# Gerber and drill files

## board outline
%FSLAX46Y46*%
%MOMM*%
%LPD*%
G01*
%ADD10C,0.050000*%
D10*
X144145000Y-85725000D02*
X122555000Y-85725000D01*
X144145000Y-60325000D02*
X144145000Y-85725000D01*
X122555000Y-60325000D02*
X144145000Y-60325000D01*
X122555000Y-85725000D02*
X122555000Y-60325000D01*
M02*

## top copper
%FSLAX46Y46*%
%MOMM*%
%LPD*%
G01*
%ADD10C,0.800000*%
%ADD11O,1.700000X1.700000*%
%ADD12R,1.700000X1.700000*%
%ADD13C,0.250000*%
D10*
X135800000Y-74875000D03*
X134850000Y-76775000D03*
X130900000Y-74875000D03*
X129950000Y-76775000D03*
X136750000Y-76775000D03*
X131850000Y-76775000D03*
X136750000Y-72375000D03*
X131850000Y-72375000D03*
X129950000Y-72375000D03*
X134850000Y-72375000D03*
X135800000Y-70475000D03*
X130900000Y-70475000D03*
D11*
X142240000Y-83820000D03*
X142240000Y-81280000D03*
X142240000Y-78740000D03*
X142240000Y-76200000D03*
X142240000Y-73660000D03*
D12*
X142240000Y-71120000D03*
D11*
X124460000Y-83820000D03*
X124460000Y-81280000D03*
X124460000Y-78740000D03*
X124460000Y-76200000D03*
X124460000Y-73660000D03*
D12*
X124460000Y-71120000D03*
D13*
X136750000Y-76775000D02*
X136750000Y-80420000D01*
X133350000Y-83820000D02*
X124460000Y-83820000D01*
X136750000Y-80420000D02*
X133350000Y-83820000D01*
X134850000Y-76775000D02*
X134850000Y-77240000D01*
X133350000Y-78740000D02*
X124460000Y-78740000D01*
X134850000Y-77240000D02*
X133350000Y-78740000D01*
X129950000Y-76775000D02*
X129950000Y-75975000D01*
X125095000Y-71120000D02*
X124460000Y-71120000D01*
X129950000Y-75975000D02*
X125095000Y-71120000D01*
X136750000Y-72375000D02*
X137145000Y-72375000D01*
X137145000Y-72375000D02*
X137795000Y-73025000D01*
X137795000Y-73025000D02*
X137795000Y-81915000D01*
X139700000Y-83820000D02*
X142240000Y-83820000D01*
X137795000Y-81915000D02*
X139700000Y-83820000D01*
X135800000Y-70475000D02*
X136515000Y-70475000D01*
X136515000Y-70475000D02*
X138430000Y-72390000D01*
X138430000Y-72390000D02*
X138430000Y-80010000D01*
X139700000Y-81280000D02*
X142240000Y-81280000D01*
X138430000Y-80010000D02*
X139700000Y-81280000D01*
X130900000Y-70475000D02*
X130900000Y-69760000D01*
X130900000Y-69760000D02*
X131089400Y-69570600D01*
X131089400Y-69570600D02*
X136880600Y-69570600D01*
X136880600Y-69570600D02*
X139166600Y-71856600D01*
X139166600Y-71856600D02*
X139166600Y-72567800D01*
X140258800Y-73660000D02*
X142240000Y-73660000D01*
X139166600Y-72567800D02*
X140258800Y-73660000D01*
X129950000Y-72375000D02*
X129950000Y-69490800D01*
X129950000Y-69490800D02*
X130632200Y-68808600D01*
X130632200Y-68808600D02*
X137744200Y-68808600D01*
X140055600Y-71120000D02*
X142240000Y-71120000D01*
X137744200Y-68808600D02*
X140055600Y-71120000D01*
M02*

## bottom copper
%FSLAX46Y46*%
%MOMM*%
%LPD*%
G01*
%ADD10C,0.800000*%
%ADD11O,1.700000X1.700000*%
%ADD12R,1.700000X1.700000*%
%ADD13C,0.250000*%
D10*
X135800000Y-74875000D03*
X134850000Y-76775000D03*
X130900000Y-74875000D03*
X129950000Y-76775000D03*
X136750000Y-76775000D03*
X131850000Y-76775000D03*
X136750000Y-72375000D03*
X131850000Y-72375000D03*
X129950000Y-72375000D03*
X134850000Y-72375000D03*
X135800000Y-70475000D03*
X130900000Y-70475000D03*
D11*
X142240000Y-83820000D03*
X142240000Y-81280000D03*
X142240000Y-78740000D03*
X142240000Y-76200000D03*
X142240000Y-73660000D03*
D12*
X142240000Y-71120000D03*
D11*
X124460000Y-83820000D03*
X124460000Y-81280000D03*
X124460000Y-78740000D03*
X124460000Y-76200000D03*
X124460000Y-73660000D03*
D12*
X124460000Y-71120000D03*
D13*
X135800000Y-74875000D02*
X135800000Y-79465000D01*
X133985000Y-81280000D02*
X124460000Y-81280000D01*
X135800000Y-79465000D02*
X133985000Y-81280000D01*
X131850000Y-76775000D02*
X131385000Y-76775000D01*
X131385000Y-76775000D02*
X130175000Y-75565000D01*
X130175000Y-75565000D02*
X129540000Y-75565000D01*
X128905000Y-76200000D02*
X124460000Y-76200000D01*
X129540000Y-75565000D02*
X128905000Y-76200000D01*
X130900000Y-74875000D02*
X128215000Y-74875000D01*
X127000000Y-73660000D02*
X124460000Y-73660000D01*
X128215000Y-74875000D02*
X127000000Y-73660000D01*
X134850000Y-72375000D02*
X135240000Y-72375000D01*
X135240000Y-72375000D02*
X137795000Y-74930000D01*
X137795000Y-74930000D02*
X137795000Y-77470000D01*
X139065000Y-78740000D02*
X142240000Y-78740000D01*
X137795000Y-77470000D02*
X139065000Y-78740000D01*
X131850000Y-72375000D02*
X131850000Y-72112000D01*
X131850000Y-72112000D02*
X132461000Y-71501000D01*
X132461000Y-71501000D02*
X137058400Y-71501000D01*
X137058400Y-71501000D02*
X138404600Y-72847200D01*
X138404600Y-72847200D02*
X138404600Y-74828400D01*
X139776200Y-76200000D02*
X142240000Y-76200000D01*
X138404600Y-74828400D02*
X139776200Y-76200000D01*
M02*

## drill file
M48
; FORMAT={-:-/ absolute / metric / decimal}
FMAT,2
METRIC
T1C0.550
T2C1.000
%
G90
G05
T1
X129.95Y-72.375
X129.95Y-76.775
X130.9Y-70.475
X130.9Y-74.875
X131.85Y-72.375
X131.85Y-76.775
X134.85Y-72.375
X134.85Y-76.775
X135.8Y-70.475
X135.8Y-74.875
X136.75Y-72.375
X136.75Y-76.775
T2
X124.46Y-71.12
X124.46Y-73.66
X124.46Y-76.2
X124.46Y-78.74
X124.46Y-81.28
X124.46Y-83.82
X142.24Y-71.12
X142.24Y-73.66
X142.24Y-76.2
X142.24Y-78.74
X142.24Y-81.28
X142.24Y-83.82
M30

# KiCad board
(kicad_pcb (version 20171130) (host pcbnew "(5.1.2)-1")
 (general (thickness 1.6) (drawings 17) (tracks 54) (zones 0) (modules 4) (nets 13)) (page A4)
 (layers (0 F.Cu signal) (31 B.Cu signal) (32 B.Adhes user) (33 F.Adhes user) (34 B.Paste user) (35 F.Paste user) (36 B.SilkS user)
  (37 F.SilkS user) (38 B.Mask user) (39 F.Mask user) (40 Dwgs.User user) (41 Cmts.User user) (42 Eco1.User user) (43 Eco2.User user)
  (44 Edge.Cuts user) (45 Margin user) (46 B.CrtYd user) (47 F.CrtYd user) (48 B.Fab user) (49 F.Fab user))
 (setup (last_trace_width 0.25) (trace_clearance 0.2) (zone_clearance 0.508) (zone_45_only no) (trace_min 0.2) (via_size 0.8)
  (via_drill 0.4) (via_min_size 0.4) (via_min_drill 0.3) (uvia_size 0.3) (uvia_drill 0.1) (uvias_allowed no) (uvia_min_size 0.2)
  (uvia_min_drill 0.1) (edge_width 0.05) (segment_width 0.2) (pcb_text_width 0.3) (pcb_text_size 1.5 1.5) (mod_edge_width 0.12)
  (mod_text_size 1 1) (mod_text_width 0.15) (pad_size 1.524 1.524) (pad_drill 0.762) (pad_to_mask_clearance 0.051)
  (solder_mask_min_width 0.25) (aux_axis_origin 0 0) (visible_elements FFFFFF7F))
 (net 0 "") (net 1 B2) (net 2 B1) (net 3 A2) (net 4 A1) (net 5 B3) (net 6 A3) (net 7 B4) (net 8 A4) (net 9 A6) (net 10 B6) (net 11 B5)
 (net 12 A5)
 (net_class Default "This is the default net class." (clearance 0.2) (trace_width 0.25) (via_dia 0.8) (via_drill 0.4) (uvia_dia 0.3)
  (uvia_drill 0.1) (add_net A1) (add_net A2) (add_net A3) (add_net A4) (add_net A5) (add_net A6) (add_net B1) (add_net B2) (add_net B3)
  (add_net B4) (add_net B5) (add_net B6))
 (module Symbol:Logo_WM (layer F.Cu) (at 125.095 64.77 270)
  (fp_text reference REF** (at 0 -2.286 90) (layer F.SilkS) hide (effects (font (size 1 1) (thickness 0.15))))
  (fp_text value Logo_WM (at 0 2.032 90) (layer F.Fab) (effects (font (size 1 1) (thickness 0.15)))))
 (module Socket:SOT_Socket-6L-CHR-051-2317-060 (layer F.Cu) (at 133.35 73.025)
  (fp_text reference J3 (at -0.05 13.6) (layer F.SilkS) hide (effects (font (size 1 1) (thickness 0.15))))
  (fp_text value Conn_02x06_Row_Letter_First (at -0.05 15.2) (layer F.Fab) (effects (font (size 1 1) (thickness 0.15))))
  (pad b2 thru_hole circle (at 2.45 1.85) (size 0.8 0.8) (drill 0.55) (layers *.Cu *.Mask) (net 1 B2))
  (pad b1 thru_hole circle (at 1.5 3.75) (size 0.8 0.8) (drill 0.55) (layers *.Cu *.Mask) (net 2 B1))
  (pad a2 thru_hole circle (at -2.45 1.85) (size 0.8 0.8) (drill 0.55) (layers *.Cu *.Mask) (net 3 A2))
  (pad a1 thru_hole circle (at -3.4 3.75) (size 0.8 0.8) (drill 0.55) (layers *.Cu *.Mask) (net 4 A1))
  (pad b3 thru_hole circle (at 3.4 3.75) (size 0.8 0.8) (drill 0.55) (layers *.Cu *.Mask) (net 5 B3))
  (pad a3 thru_hole circle (at -1.5 3.75) (size 0.8 0.8) (drill 0.55) (layers *.Cu *.Mask) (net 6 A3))
  (pad b4 thru_hole circle (at 3.4 -0.65) (size 0.8 0.8) (drill 0.55) (layers *.Cu *.Mask) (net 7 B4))
  (pad a4 thru_hole circle (at -1.5 -0.65) (size 0.8 0.8) (drill 0.55) (layers *.Cu *.Mask) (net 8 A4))
  (pad a6 thru_hole circle (at -3.4 -0.65) (size 0.8 0.8) (drill 0.55) (layers *.Cu *.Mask) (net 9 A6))
  (pad b6 thru_hole circle (at 1.5 -0.65) (size 0.8 0.8) (drill 0.55) (layers *.Cu *.Mask) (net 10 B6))
  (pad b5 thru_hole circle (at 2.45 -2.55) (size 0.8 0.8) (drill 0.55) (layers *.Cu *.Mask) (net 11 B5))
  (pad a5 thru_hole circle (at -2.45 -2.55) (size 0.8 0.8) (drill 0.55) (layers *.Cu *.Mask) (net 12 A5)))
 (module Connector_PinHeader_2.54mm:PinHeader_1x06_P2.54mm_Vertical (layer B.Cu) (at 142.24 71.12 180)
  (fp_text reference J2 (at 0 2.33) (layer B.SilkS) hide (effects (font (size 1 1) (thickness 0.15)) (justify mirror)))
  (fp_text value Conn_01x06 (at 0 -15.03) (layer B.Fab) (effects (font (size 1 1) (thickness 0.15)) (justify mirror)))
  (pad 6 thru_hole oval (at 0 -12.7 180) (size 1.7 1.7) (drill 1) (layers *.Cu *.Mask) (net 7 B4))
  (pad 5 thru_hole oval (at 0 -10.16 180) (size 1.7 1.7) (drill 1) (layers *.Cu *.Mask) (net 11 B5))
  (pad 4 thru_hole oval (at 0 -7.62 180) (size 1.7 1.7) (drill 1) (layers *.Cu *.Mask) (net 10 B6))
  (pad 3 thru_hole oval (at 0 -5.08 180) (size 1.7 1.7) (drill 1) (layers *.Cu *.Mask) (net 8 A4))
  (pad 2 thru_hole oval (at 0 -2.54 180) (size 1.7 1.7) (drill 1) (layers *.Cu *.Mask) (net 12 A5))
  (pad 1 thru_hole rect (at 0 0 180) (size 1.7 1.7) (drill 1) (layers *.Cu *.Mask) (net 9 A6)))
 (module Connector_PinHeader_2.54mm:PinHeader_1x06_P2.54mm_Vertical (layer B.Cu) (at 124.46 71.12 180)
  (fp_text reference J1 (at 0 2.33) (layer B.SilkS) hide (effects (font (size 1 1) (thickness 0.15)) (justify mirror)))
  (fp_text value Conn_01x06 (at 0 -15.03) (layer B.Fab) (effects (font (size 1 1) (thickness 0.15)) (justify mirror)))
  (pad 6 thru_hole oval (at 0 -12.7 180) (size 1.7 1.7) (drill 1) (layers *.Cu *.Mask) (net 5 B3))
  (pad 5 thru_hole oval (at 0 -10.16 180) (size 1.7 1.7) (drill 1) (layers *.Cu *.Mask) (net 1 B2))
  (pad 4 thru_hole oval (at 0 -7.62 180) (size 1.7 1.7) (drill 1) (layers *.Cu *.Mask) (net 2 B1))
  (pad 3 thru_hole oval (at 0 -5.08 180) (size 1.7 1.7) (drill 1) (layers *.Cu *.Mask) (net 6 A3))
  (pad 2 thru_hole oval (at 0 -2.54 180) (size 1.7 1.7) (drill 1) (layers *.Cu *.Mask) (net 3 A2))
  (pad 1 thru_hole rect (at 0 0 180) (size 1.7 1.7) (drill 1) (layers *.Cu *.Mask) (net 4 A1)))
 (gr_line (start 144.145 85.725) (end 122.555 85.725) (layer Edge.Cuts) (width 0.05))
 (gr_line (start 144.145 60.325) (end 144.145 85.725) (layer Edge.Cuts) (width 0.05))
 (gr_line (start 122.555 60.325) (end 144.145 60.325) (layer Edge.Cuts) (width 0.05))
 (gr_line (start 122.555 85.725) (end 122.555 60.325) (layer Edge.Cuts) (width 0.05))
 (segment (start 136.75 76.775) (end 136.75 80.42) (width 0.25) (layer F.Cu) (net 5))
 (segment (start 133.35 83.82) (end 124.46 83.82) (width 0.25) (layer F.Cu) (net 5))
 (segment (start 136.75 80.42) (end 133.35 83.82) (width 0.25) (layer F.Cu) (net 5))
 (segment (start 135.8 74.875) (end 135.8 79.465) (width 0.25) (layer B.Cu) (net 1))
 (segment (start 133.985 81.28) (end 124.46 81.28) (width 0.25) (layer B.Cu) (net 1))
 (segment (start 135.8 79.465) (end 133.985 81.28) (width 0.25) (layer B.Cu) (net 1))
 (segment (start 134.85 76.775) (end 134.85 77.24) (width 0.25) (layer F.Cu) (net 2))
 (segment (start 133.35 78.74) (end 124.46 78.74) (width 0.25) (layer F.Cu) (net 2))
 (segment (start 134.85 77.24) (end 133.35 78.74) (width 0.25) (layer F.Cu) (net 2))
 (segment (start 131.85 76.775) (end 131.385 76.775) (width 0.25) (layer B.Cu) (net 6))
 (segment (start 131.385 76.775) (end 130.175 75.565) (width 0.25) (layer B.Cu) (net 6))
 (segment (start 130.175 75.565) (end 129.54 75.565) (width 0.25) (layer B.Cu) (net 6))
 (segment (start 128.905 76.2) (end 124.46 76.2) (width 0.25) (layer B.Cu) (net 6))
 (segment (start 129.54 75.565) (end 128.905 76.2) (width 0.25) (layer B.Cu) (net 6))
 (segment (start 130.9 74.875) (end 128.215 74.875) (width 0.25) (layer B.Cu) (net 3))
 (segment (start 127 73.66) (end 124.46 73.66) (width 0.25) (layer B.Cu) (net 3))
 (segment (start 128.215 74.875) (end 127 73.66) (width 0.25) (layer B.Cu) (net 3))
 (segment (start 129.95 76.775) (end 129.95 75.975) (width 0.25) (layer F.Cu) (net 4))
 (segment (start 125.095 71.12) (end 124.46 71.12) (width 0.25) (layer F.Cu) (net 4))
 (segment (start 129.95 75.975) (end 125.095 71.12) (width 0.25) (layer F.Cu) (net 4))
 (segment (start 136.75 72.375) (end 137.145 72.375) (width 0.25) (layer F.Cu) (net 7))
 (segment (start 137.145 72.375) (end 137.795 73.025) (width 0.25) (layer F.Cu) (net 7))
 (segment (start 137.795 73.025) (end 137.795 81.915) (width 0.25) (layer F.Cu) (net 7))
 (segment (start 139.7 83.82) (end 142.24 83.82) (width 0.25) (layer F.Cu) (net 7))
 (segment (start 137.795 81.915) (end 139.7 83.82) (width 0.25) (layer F.Cu) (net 7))
 (segment (start 135.8 70.475) (end 136.515 70.475) (width 0.25) (layer F.Cu) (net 11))
 (segment (start 136.515 70.475) (end 138.43 72.39) (width 0.25) (layer F.Cu) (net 11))
 (segment (start 138.43 72.39) (end 138.43 80.01) (width 0.25) (layer F.Cu) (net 11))
 (segment (start 139.7 81.28) (end 142.24 81.28) (width 0.25) (layer F.Cu) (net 11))
 (segment (start 138.43 80.01) (end 139.7 81.28) (width 0.25) (layer F.Cu) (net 11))
 (segment (start 134.85 72.375) (end 135.24 72.375) (width 0.25) (layer B.Cu) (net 10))
 (segment (start 135.24 72.375) (end 137.795 74.93) (width 0.25) (layer B.Cu) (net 10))
 (segment (start 137.795 74.93) (end 137.795 77.47) (width 0.25) (layer B.Cu) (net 10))
 (segment (start 139.065 78.74) (end 142.24 78.74) (width 0.25) (layer B.Cu) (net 10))
 (segment (start 137.795 77.47) (end 139.065 78.74) (width 0.25) (layer B.Cu) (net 10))
 (segment (start 131.85 72.375) (end 131.85 72.112) (width 0.25) (layer B.Cu) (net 8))
 (segment (start 131.85 72.112) (end 132.461 71.501) (width 0.25) (layer B.Cu) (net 8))
 (segment (start 132.461 71.501) (end 137.0584 71.501) (width 0.25) (layer B.Cu) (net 8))
 (segment (start 137.0584 71.501) (end 138.4046 72.8472) (width 0.25) (layer B.Cu) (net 8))
 (segment (start 138.4046 72.8472) (end 138.4046 74.8284) (width 0.25) (layer B.Cu) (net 8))
 (segment (start 139.7762 76.2) (end 142.24 76.2) (width 0.25) (layer B.Cu) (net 8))
 (segment (start 138.4046 74.8284) (end 139.7762 76.2) (width 0.25) (layer B.Cu) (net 8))
 (segment (start 130.9 70.475) (end 130.9 69.76) (width 0.25) (layer F.Cu) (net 12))
 (segment (start 130.9 69.76) (end 131.0894 69.5706) (width 0.25) (layer F.Cu) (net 12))
 (segment (start 131.0894 69.5706) (end 136.8806 69.5706) (width 0.25) (layer F.Cu) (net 12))
 (segment (start 136.8806 69.5706) (end 139.1666 71.8566) (width 0.25) (layer F.Cu) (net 12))
 (segment (start 139.1666 71.8566) (end 139.1666 72.5678) (width 0.25) (layer F.Cu) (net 12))
 (segment (start 140.2588 73.66) (end 142.24 73.66) (width 0.25) (layer F.Cu) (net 12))
 (segment (start 139.1666 72.5678) (end 140.2588 73.66) (width 0.25) (layer F.Cu) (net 12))
 (segment (start 129.95 72.375) (end 129.95 69.4908) (width 0.25) (layer F.Cu) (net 9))
 (segment (start 129.95 69.4908) (end 130.6322 68.8086) (width 0.25) (layer F.Cu) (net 9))
 (segment (start 130.6322 68.8086) (end 137.7442 68.8086) (width 0.25) (layer F.Cu) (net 9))
 (segment (start 140.0556 71.12) (end 142.24 71.12) (width 0.25) (layer F.Cu) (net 9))
 (segment (start 137.7442 68.8086) (end 140.0556 71.12) (width 0.25) (layer F.Cu) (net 9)))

